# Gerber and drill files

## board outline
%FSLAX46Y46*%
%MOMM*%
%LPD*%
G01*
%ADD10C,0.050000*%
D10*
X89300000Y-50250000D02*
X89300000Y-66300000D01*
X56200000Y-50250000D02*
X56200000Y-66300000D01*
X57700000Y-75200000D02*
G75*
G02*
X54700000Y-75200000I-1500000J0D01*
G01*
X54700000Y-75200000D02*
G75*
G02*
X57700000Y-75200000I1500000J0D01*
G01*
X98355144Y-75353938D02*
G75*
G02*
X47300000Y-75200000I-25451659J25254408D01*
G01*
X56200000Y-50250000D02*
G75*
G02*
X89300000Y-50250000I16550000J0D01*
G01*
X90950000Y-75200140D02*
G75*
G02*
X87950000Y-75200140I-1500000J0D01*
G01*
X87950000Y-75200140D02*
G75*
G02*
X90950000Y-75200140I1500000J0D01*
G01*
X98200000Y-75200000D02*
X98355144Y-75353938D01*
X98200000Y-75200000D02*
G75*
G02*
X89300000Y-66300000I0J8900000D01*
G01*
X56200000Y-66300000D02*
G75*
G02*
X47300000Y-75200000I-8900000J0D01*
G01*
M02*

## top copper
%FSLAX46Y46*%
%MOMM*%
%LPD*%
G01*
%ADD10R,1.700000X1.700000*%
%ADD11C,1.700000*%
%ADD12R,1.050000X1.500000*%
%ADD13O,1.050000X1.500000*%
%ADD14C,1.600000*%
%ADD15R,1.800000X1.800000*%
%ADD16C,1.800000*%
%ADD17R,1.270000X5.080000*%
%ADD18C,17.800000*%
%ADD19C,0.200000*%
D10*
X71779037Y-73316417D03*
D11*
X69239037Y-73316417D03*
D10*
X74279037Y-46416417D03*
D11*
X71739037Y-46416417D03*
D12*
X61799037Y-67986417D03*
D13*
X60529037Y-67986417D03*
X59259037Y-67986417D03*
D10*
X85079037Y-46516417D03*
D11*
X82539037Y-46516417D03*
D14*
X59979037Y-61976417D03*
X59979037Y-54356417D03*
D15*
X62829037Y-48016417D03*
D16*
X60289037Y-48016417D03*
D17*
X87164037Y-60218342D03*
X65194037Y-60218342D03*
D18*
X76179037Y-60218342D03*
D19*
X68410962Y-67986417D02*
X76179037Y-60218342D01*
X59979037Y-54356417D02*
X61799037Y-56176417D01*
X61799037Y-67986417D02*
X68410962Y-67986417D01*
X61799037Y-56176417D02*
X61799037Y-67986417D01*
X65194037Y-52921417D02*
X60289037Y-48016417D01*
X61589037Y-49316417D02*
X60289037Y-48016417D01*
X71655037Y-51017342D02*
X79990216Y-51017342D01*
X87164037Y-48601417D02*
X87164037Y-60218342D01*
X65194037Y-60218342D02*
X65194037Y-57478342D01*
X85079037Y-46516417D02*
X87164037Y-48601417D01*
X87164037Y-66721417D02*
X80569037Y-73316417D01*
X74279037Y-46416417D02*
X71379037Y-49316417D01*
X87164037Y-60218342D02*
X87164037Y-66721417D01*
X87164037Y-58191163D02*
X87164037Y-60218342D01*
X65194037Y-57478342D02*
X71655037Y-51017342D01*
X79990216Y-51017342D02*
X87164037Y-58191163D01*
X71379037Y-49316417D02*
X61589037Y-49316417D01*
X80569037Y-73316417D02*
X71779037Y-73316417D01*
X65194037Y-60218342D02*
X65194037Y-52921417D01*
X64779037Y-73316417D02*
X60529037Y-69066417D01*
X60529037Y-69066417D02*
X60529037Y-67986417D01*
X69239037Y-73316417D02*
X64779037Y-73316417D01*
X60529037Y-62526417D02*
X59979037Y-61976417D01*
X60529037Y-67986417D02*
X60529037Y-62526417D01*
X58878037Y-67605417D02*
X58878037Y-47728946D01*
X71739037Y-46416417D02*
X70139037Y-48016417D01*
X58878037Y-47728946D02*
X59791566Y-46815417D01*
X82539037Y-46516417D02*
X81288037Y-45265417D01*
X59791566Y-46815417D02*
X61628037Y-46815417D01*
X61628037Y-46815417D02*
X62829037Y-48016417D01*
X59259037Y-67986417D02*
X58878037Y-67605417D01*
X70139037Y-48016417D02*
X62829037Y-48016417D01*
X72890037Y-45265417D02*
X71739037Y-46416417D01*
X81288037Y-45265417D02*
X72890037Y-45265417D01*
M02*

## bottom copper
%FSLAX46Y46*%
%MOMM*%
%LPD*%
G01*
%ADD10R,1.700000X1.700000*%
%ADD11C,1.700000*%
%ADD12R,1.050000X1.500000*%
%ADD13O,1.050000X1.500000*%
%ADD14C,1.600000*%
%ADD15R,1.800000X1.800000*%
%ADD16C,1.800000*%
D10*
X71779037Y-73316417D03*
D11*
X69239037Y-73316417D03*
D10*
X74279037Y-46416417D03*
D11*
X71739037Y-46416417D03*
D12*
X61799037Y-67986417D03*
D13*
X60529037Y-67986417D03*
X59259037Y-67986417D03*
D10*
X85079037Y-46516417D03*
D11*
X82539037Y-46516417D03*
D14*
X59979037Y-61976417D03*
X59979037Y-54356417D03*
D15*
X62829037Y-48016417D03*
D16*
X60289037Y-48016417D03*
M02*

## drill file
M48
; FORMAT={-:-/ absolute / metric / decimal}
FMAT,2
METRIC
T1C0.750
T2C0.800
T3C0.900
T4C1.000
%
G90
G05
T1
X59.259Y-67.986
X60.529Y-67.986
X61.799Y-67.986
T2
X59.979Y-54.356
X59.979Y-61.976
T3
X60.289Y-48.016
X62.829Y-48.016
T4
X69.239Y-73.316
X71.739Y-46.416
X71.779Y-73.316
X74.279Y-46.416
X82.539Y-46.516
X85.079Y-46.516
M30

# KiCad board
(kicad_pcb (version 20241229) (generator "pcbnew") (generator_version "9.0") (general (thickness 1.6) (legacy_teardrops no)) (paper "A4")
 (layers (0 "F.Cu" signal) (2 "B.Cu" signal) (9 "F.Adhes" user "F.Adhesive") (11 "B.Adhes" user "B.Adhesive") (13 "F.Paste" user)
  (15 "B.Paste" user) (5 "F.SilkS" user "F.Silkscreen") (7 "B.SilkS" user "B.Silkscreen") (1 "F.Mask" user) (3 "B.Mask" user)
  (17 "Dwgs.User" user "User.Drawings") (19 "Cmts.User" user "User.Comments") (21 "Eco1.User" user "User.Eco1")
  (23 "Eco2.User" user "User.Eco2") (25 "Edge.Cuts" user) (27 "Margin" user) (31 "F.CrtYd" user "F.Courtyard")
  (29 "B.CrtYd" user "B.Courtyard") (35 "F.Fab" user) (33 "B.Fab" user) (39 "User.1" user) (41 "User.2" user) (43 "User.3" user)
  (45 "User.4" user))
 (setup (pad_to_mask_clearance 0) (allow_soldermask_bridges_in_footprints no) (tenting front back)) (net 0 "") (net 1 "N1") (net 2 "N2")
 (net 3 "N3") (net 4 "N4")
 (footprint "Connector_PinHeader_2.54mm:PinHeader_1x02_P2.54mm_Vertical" (layer "F.Cu") (at 71.779037 73.316417 -90)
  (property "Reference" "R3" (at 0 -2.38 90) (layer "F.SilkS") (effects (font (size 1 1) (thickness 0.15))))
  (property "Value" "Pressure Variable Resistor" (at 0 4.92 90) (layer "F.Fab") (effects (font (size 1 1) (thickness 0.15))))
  (pad "1" thru_hole rect (at 0 0 270) (size 1.7 1.7) (drill 1) (layers "*.Cu" "*.Mask") (remove_unused_layers no) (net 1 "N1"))
  (pad "2" thru_hole circle (at 0 2.54 270) (size 1.7 1.7) (drill 1) (layers "*.Cu" "*.Mask") (remove_unused_layers no) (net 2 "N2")))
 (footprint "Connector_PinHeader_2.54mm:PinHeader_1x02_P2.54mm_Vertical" (layer "F.Cu") (at 74.279037 46.416417 -90)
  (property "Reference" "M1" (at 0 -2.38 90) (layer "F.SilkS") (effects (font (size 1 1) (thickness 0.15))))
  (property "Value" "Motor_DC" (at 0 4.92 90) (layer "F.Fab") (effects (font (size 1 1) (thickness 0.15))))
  (pad "1" thru_hole rect (at 0 0 270) (size 1.7 1.7) (drill 1) (layers "*.Cu" "*.Mask") (remove_unused_layers no) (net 1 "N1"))
  (pad "2" thru_hole circle (at 0 2.54 270) (size 1.7 1.7) (drill 1) (layers "*.Cu" "*.Mask") (remove_unused_layers no) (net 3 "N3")))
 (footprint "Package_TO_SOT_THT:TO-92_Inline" (layer "F.Cu") (at 61.799037 67.986417 180)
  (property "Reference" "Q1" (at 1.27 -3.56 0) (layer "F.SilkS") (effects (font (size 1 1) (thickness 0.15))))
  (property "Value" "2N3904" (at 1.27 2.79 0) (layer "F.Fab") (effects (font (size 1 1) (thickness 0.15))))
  (pad "1" thru_hole rect (at 0 0 180) (size 1.05 1.5) (drill 0.75) (layers "*.Cu" "*.Mask") (remove_unused_layers no) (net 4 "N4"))
  (pad "2" thru_hole oval (at 1.27 0 180) (size 1.05 1.5) (drill 0.75) (layers "*.Cu" "*.Mask") (remove_unused_layers no) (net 2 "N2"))
  (pad "3" thru_hole oval (at 2.54 0 180) (size 1.05 1.5) (drill 0.75) (layers "*.Cu" "*.Mask") (remove_unused_layers no) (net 3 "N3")))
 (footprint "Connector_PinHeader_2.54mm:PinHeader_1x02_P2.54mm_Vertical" (layer "F.Cu") (at 85.079037 46.516417 -90)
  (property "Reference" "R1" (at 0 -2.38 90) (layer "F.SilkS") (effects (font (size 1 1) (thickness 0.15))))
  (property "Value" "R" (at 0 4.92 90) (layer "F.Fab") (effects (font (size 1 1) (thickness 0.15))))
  (pad "1" thru_hole rect (at 0 0 270) (size 1.7 1.7) (drill 1) (layers "*.Cu" "*.Mask") (remove_unused_layers no) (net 1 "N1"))
  (pad "2" thru_hole circle (at 0 2.54 270) (size 1.7 1.7) (drill 1) (layers "*.Cu" "*.Mask") (remove_unused_layers no) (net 3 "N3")))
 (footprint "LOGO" (layer "F.Cu") (at 74.6 79.4)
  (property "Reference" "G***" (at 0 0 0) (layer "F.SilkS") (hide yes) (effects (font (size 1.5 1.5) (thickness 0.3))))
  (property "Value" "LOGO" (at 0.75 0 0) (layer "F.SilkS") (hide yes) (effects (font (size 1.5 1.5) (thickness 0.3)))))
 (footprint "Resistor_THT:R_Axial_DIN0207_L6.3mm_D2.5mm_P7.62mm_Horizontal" (layer "F.Cu") (at 59.979037 61.976417 90)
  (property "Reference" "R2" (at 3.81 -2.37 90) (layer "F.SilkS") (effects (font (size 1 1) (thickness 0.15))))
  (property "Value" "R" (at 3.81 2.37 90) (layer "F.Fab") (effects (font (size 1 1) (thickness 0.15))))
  (pad "1" thru_hole circle (at 0 0 90) (size 1.6 1.6) (drill 0.8) (layers "*.Cu" "*.Mask") (remove_unused_layers no) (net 2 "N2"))
  (pad "2" thru_hole circle (at 7.62 0 90) (size 1.6 1.6) (drill 0.8) (layers "*.Cu" "*.Mask") (remove_unused_layers no) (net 4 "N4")))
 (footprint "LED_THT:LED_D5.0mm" (layer "F.Cu") (at 62.829037 48.016417 180)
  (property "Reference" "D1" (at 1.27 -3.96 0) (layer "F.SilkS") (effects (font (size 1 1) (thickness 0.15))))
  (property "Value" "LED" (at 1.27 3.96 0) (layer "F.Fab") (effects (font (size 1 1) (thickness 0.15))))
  (pad "1" thru_hole rect (at 0 0 180) (size 1.8 1.8) (drill 0.9) (layers "*.Cu" "*.Mask") (remove_unused_layers no) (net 3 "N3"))
  (pad "2" thru_hole circle (at 2.54 0 180) (size 1.8 1.8) (drill 0.9) (layers "*.Cu" "*.Mask") (remove_unused_layers no) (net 1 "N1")))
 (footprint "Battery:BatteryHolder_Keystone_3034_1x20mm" (layer "F.Cu") (at 76.179037 60.218342 180)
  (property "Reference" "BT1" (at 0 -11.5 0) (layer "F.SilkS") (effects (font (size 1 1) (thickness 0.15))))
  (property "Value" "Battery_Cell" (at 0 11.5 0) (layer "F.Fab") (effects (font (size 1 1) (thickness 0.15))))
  (pad "1" smd rect (at -10.985 0 180) (size 1.27 5.08) (layers "F.Cu" "F.Mask" "F.Paste") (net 1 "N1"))
  (pad "1" smd rect (at 10.985 0 180) (size 1.27 5.08) (layers "F.Cu" "F.Mask" "F.Paste") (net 1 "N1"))
  (pad "2" smd circle (at 0 0 180) (size 17.8 17.8) (layers "F.Cu" "F.Mask") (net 4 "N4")))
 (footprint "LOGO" (layer "B.Cu") (at 72.959069 52.06647 180)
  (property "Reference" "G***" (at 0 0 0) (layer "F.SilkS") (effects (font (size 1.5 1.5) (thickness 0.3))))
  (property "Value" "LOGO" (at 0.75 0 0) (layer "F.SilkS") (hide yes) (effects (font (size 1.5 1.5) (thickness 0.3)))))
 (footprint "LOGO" (layer "B.Cu") (at 72.68318 78.185004 180)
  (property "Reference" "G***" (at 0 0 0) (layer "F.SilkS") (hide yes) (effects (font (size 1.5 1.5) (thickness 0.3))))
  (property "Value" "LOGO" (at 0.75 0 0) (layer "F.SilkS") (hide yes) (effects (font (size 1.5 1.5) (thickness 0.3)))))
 (gr_line (start 89.3 50.25) (end 89.3 66.3) (stroke (width 0.05) (type solid)) (layer "Edge.Cuts"))
 (gr_line (start 56.2 50.25) (end 56.2 66.3) (stroke (width 0.05) (type solid)) (layer "Edge.Cuts"))
 (gr_circle (center 56.2 75.2) (end 57.7 75.2) (stroke (width 0.05) (type default)) (fill no) (layer "Edge.Cuts"))
 (gr_arc (start 98.355144 75.353938) (mid 72.795379 85.954242) (end 47.3 75.2) (stroke (width 0.05) (type solid)) (layer "Edge.Cuts"))
 (gr_arc (start 56.2 50.25) (mid 72.75 33.7) (end 89.3 50.25) (stroke (width 0.05) (type default)) (layer "Edge.Cuts"))
 (gr_circle (center 89.45 75.20014) (end 90.95 75.20014) (stroke (width 0.05) (type solid)) (fill no) (layer "Edge.Cuts"))
 (gr_line (start 98.2 75.2) (end 98.355144 75.353938) (stroke (width 0.05) (type default)) (layer "Edge.Cuts"))
 (gr_arc (start 98.2 75.2) (mid 91.90675 72.59325) (end 89.3 66.3) (stroke (width 0.05) (type default)) (layer "Edge.Cuts"))
 (gr_arc (start 56.2 66.3) (mid 53.59325 72.59325) (end 47.3 75.2) (stroke (width 0.05) (type solid)) (layer "Edge.Cuts"))
 (segment (start 68.410962 67.986417) (end 76.179037 60.218342) (width 0.2) (layer "F.Cu") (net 4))
 (segment (start 59.979037 54.356417) (end 61.799037 56.176417) (width 0.2) (layer "F.Cu") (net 4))
 (segment (start 61.799037 67.986417) (end 68.410962 67.986417) (width 0.2) (layer "F.Cu") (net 4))
 (segment (start 61.799037 56.176417) (end 61.799037 67.986417) (width 0.2) (layer "F.Cu") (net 4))
 (segment (start 65.194037 52.921417) (end 60.289037 48.016417) (width 0.2) (layer "F.Cu") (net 1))
 (segment (start 61.589037 49.316417) (end 60.289037 48.016417) (width 0.2) (layer "F.Cu") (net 1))
 (segment (start 71.655037 51.017342) (end 79.990216 51.017342) (width 0.2) (layer "F.Cu") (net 1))
 (segment (start 87.164037 48.601417) (end 87.164037 60.218342) (width 0.2) (layer "F.Cu") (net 1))
 (segment (start 65.194037 60.218342) (end 65.194037 57.478342) (width 0.2) (layer "F.Cu") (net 1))
 (segment (start 85.079037 46.516417) (end 87.164037 48.601417) (width 0.2) (layer "F.Cu") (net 1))
 (segment (start 87.164037 66.721417) (end 80.569037 73.316417) (width 0.2) (layer "F.Cu") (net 1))
 (segment (start 74.279037 46.416417) (end 71.379037 49.316417) (width 0.2) (layer "F.Cu") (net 1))
 (segment (start 87.164037 60.218342) (end 87.164037 66.721417) (width 0.2) (layer "F.Cu") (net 1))
 (segment (start 87.164037 58.191163) (end 87.164037 60.218342) (width 0.2) (layer "F.Cu") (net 1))
 (segment (start 65.194037 57.478342) (end 71.655037 51.017342) (width 0.2) (layer "F.Cu") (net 1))
 (segment (start 79.990216 51.017342) (end 87.164037 58.191163) (width 0.2) (layer "F.Cu") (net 1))
 (segment (start 71.379037 49.316417) (end 61.589037 49.316417) (width 0.2) (layer "F.Cu") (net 1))
 (segment (start 80.569037 73.316417) (end 71.779037 73.316417) (width 0.2) (layer "F.Cu") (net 1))
 (segment (start 65.194037 60.218342) (end 65.194037 52.921417) (width 0.2) (layer "F.Cu") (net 1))
 (segment (start 64.779037 73.316417) (end 60.529037 69.066417) (width 0.2) (layer "F.Cu") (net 2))
 (segment (start 60.529037 69.066417) (end 60.529037 67.986417) (width 0.2) (layer "F.Cu") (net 2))
 (segment (start 69.239037 73.316417) (end 64.779037 73.316417) (width 0.2) (layer "F.Cu") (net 2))
 (segment (start 60.529037 62.526417) (end 59.979037 61.976417) (width 0.2) (layer "F.Cu") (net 2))
 (segment (start 60.529037 67.986417) (end 60.529037 62.526417) (width 0.2) (layer "F.Cu") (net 2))
 (segment (start 58.878037 67.605417) (end 58.878037 47.728946) (width 0.2) (layer "F.Cu") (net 3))
 (segment (start 71.739037 46.416417) (end 70.139037 48.016417) (width 0.2) (layer "F.Cu") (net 3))
 (segment (start 58.878037 47.728946) (end 59.791566 46.815417) (width 0.2) (layer "F.Cu") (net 3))
 (segment (start 82.539037 46.516417) (end 81.288037 45.265417) (width 0.2) (layer "F.Cu") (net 3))
 (segment (start 59.791566 46.815417) (end 61.628037 46.815417) (width 0.2) (layer "F.Cu") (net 3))
 (segment (start 61.628037 46.815417) (end 62.829037 48.016417) (width 0.2) (layer "F.Cu") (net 3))
 (segment (start 59.259037 67.986417) (end 58.878037 67.605417) (width 0.2) (layer "F.Cu") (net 3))
 (segment (start 70.139037 48.016417) (end 62.829037 48.016417) (width 0.2) (layer "F.Cu") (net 3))
 (segment (start 72.890037 45.265417) (end 71.739037 46.416417) (width 0.2) (layer "F.Cu") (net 3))
 (segment (start 81.288037 45.265417) (end 72.890037 45.265417) (width 0.2) (layer "F.Cu") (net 3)))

